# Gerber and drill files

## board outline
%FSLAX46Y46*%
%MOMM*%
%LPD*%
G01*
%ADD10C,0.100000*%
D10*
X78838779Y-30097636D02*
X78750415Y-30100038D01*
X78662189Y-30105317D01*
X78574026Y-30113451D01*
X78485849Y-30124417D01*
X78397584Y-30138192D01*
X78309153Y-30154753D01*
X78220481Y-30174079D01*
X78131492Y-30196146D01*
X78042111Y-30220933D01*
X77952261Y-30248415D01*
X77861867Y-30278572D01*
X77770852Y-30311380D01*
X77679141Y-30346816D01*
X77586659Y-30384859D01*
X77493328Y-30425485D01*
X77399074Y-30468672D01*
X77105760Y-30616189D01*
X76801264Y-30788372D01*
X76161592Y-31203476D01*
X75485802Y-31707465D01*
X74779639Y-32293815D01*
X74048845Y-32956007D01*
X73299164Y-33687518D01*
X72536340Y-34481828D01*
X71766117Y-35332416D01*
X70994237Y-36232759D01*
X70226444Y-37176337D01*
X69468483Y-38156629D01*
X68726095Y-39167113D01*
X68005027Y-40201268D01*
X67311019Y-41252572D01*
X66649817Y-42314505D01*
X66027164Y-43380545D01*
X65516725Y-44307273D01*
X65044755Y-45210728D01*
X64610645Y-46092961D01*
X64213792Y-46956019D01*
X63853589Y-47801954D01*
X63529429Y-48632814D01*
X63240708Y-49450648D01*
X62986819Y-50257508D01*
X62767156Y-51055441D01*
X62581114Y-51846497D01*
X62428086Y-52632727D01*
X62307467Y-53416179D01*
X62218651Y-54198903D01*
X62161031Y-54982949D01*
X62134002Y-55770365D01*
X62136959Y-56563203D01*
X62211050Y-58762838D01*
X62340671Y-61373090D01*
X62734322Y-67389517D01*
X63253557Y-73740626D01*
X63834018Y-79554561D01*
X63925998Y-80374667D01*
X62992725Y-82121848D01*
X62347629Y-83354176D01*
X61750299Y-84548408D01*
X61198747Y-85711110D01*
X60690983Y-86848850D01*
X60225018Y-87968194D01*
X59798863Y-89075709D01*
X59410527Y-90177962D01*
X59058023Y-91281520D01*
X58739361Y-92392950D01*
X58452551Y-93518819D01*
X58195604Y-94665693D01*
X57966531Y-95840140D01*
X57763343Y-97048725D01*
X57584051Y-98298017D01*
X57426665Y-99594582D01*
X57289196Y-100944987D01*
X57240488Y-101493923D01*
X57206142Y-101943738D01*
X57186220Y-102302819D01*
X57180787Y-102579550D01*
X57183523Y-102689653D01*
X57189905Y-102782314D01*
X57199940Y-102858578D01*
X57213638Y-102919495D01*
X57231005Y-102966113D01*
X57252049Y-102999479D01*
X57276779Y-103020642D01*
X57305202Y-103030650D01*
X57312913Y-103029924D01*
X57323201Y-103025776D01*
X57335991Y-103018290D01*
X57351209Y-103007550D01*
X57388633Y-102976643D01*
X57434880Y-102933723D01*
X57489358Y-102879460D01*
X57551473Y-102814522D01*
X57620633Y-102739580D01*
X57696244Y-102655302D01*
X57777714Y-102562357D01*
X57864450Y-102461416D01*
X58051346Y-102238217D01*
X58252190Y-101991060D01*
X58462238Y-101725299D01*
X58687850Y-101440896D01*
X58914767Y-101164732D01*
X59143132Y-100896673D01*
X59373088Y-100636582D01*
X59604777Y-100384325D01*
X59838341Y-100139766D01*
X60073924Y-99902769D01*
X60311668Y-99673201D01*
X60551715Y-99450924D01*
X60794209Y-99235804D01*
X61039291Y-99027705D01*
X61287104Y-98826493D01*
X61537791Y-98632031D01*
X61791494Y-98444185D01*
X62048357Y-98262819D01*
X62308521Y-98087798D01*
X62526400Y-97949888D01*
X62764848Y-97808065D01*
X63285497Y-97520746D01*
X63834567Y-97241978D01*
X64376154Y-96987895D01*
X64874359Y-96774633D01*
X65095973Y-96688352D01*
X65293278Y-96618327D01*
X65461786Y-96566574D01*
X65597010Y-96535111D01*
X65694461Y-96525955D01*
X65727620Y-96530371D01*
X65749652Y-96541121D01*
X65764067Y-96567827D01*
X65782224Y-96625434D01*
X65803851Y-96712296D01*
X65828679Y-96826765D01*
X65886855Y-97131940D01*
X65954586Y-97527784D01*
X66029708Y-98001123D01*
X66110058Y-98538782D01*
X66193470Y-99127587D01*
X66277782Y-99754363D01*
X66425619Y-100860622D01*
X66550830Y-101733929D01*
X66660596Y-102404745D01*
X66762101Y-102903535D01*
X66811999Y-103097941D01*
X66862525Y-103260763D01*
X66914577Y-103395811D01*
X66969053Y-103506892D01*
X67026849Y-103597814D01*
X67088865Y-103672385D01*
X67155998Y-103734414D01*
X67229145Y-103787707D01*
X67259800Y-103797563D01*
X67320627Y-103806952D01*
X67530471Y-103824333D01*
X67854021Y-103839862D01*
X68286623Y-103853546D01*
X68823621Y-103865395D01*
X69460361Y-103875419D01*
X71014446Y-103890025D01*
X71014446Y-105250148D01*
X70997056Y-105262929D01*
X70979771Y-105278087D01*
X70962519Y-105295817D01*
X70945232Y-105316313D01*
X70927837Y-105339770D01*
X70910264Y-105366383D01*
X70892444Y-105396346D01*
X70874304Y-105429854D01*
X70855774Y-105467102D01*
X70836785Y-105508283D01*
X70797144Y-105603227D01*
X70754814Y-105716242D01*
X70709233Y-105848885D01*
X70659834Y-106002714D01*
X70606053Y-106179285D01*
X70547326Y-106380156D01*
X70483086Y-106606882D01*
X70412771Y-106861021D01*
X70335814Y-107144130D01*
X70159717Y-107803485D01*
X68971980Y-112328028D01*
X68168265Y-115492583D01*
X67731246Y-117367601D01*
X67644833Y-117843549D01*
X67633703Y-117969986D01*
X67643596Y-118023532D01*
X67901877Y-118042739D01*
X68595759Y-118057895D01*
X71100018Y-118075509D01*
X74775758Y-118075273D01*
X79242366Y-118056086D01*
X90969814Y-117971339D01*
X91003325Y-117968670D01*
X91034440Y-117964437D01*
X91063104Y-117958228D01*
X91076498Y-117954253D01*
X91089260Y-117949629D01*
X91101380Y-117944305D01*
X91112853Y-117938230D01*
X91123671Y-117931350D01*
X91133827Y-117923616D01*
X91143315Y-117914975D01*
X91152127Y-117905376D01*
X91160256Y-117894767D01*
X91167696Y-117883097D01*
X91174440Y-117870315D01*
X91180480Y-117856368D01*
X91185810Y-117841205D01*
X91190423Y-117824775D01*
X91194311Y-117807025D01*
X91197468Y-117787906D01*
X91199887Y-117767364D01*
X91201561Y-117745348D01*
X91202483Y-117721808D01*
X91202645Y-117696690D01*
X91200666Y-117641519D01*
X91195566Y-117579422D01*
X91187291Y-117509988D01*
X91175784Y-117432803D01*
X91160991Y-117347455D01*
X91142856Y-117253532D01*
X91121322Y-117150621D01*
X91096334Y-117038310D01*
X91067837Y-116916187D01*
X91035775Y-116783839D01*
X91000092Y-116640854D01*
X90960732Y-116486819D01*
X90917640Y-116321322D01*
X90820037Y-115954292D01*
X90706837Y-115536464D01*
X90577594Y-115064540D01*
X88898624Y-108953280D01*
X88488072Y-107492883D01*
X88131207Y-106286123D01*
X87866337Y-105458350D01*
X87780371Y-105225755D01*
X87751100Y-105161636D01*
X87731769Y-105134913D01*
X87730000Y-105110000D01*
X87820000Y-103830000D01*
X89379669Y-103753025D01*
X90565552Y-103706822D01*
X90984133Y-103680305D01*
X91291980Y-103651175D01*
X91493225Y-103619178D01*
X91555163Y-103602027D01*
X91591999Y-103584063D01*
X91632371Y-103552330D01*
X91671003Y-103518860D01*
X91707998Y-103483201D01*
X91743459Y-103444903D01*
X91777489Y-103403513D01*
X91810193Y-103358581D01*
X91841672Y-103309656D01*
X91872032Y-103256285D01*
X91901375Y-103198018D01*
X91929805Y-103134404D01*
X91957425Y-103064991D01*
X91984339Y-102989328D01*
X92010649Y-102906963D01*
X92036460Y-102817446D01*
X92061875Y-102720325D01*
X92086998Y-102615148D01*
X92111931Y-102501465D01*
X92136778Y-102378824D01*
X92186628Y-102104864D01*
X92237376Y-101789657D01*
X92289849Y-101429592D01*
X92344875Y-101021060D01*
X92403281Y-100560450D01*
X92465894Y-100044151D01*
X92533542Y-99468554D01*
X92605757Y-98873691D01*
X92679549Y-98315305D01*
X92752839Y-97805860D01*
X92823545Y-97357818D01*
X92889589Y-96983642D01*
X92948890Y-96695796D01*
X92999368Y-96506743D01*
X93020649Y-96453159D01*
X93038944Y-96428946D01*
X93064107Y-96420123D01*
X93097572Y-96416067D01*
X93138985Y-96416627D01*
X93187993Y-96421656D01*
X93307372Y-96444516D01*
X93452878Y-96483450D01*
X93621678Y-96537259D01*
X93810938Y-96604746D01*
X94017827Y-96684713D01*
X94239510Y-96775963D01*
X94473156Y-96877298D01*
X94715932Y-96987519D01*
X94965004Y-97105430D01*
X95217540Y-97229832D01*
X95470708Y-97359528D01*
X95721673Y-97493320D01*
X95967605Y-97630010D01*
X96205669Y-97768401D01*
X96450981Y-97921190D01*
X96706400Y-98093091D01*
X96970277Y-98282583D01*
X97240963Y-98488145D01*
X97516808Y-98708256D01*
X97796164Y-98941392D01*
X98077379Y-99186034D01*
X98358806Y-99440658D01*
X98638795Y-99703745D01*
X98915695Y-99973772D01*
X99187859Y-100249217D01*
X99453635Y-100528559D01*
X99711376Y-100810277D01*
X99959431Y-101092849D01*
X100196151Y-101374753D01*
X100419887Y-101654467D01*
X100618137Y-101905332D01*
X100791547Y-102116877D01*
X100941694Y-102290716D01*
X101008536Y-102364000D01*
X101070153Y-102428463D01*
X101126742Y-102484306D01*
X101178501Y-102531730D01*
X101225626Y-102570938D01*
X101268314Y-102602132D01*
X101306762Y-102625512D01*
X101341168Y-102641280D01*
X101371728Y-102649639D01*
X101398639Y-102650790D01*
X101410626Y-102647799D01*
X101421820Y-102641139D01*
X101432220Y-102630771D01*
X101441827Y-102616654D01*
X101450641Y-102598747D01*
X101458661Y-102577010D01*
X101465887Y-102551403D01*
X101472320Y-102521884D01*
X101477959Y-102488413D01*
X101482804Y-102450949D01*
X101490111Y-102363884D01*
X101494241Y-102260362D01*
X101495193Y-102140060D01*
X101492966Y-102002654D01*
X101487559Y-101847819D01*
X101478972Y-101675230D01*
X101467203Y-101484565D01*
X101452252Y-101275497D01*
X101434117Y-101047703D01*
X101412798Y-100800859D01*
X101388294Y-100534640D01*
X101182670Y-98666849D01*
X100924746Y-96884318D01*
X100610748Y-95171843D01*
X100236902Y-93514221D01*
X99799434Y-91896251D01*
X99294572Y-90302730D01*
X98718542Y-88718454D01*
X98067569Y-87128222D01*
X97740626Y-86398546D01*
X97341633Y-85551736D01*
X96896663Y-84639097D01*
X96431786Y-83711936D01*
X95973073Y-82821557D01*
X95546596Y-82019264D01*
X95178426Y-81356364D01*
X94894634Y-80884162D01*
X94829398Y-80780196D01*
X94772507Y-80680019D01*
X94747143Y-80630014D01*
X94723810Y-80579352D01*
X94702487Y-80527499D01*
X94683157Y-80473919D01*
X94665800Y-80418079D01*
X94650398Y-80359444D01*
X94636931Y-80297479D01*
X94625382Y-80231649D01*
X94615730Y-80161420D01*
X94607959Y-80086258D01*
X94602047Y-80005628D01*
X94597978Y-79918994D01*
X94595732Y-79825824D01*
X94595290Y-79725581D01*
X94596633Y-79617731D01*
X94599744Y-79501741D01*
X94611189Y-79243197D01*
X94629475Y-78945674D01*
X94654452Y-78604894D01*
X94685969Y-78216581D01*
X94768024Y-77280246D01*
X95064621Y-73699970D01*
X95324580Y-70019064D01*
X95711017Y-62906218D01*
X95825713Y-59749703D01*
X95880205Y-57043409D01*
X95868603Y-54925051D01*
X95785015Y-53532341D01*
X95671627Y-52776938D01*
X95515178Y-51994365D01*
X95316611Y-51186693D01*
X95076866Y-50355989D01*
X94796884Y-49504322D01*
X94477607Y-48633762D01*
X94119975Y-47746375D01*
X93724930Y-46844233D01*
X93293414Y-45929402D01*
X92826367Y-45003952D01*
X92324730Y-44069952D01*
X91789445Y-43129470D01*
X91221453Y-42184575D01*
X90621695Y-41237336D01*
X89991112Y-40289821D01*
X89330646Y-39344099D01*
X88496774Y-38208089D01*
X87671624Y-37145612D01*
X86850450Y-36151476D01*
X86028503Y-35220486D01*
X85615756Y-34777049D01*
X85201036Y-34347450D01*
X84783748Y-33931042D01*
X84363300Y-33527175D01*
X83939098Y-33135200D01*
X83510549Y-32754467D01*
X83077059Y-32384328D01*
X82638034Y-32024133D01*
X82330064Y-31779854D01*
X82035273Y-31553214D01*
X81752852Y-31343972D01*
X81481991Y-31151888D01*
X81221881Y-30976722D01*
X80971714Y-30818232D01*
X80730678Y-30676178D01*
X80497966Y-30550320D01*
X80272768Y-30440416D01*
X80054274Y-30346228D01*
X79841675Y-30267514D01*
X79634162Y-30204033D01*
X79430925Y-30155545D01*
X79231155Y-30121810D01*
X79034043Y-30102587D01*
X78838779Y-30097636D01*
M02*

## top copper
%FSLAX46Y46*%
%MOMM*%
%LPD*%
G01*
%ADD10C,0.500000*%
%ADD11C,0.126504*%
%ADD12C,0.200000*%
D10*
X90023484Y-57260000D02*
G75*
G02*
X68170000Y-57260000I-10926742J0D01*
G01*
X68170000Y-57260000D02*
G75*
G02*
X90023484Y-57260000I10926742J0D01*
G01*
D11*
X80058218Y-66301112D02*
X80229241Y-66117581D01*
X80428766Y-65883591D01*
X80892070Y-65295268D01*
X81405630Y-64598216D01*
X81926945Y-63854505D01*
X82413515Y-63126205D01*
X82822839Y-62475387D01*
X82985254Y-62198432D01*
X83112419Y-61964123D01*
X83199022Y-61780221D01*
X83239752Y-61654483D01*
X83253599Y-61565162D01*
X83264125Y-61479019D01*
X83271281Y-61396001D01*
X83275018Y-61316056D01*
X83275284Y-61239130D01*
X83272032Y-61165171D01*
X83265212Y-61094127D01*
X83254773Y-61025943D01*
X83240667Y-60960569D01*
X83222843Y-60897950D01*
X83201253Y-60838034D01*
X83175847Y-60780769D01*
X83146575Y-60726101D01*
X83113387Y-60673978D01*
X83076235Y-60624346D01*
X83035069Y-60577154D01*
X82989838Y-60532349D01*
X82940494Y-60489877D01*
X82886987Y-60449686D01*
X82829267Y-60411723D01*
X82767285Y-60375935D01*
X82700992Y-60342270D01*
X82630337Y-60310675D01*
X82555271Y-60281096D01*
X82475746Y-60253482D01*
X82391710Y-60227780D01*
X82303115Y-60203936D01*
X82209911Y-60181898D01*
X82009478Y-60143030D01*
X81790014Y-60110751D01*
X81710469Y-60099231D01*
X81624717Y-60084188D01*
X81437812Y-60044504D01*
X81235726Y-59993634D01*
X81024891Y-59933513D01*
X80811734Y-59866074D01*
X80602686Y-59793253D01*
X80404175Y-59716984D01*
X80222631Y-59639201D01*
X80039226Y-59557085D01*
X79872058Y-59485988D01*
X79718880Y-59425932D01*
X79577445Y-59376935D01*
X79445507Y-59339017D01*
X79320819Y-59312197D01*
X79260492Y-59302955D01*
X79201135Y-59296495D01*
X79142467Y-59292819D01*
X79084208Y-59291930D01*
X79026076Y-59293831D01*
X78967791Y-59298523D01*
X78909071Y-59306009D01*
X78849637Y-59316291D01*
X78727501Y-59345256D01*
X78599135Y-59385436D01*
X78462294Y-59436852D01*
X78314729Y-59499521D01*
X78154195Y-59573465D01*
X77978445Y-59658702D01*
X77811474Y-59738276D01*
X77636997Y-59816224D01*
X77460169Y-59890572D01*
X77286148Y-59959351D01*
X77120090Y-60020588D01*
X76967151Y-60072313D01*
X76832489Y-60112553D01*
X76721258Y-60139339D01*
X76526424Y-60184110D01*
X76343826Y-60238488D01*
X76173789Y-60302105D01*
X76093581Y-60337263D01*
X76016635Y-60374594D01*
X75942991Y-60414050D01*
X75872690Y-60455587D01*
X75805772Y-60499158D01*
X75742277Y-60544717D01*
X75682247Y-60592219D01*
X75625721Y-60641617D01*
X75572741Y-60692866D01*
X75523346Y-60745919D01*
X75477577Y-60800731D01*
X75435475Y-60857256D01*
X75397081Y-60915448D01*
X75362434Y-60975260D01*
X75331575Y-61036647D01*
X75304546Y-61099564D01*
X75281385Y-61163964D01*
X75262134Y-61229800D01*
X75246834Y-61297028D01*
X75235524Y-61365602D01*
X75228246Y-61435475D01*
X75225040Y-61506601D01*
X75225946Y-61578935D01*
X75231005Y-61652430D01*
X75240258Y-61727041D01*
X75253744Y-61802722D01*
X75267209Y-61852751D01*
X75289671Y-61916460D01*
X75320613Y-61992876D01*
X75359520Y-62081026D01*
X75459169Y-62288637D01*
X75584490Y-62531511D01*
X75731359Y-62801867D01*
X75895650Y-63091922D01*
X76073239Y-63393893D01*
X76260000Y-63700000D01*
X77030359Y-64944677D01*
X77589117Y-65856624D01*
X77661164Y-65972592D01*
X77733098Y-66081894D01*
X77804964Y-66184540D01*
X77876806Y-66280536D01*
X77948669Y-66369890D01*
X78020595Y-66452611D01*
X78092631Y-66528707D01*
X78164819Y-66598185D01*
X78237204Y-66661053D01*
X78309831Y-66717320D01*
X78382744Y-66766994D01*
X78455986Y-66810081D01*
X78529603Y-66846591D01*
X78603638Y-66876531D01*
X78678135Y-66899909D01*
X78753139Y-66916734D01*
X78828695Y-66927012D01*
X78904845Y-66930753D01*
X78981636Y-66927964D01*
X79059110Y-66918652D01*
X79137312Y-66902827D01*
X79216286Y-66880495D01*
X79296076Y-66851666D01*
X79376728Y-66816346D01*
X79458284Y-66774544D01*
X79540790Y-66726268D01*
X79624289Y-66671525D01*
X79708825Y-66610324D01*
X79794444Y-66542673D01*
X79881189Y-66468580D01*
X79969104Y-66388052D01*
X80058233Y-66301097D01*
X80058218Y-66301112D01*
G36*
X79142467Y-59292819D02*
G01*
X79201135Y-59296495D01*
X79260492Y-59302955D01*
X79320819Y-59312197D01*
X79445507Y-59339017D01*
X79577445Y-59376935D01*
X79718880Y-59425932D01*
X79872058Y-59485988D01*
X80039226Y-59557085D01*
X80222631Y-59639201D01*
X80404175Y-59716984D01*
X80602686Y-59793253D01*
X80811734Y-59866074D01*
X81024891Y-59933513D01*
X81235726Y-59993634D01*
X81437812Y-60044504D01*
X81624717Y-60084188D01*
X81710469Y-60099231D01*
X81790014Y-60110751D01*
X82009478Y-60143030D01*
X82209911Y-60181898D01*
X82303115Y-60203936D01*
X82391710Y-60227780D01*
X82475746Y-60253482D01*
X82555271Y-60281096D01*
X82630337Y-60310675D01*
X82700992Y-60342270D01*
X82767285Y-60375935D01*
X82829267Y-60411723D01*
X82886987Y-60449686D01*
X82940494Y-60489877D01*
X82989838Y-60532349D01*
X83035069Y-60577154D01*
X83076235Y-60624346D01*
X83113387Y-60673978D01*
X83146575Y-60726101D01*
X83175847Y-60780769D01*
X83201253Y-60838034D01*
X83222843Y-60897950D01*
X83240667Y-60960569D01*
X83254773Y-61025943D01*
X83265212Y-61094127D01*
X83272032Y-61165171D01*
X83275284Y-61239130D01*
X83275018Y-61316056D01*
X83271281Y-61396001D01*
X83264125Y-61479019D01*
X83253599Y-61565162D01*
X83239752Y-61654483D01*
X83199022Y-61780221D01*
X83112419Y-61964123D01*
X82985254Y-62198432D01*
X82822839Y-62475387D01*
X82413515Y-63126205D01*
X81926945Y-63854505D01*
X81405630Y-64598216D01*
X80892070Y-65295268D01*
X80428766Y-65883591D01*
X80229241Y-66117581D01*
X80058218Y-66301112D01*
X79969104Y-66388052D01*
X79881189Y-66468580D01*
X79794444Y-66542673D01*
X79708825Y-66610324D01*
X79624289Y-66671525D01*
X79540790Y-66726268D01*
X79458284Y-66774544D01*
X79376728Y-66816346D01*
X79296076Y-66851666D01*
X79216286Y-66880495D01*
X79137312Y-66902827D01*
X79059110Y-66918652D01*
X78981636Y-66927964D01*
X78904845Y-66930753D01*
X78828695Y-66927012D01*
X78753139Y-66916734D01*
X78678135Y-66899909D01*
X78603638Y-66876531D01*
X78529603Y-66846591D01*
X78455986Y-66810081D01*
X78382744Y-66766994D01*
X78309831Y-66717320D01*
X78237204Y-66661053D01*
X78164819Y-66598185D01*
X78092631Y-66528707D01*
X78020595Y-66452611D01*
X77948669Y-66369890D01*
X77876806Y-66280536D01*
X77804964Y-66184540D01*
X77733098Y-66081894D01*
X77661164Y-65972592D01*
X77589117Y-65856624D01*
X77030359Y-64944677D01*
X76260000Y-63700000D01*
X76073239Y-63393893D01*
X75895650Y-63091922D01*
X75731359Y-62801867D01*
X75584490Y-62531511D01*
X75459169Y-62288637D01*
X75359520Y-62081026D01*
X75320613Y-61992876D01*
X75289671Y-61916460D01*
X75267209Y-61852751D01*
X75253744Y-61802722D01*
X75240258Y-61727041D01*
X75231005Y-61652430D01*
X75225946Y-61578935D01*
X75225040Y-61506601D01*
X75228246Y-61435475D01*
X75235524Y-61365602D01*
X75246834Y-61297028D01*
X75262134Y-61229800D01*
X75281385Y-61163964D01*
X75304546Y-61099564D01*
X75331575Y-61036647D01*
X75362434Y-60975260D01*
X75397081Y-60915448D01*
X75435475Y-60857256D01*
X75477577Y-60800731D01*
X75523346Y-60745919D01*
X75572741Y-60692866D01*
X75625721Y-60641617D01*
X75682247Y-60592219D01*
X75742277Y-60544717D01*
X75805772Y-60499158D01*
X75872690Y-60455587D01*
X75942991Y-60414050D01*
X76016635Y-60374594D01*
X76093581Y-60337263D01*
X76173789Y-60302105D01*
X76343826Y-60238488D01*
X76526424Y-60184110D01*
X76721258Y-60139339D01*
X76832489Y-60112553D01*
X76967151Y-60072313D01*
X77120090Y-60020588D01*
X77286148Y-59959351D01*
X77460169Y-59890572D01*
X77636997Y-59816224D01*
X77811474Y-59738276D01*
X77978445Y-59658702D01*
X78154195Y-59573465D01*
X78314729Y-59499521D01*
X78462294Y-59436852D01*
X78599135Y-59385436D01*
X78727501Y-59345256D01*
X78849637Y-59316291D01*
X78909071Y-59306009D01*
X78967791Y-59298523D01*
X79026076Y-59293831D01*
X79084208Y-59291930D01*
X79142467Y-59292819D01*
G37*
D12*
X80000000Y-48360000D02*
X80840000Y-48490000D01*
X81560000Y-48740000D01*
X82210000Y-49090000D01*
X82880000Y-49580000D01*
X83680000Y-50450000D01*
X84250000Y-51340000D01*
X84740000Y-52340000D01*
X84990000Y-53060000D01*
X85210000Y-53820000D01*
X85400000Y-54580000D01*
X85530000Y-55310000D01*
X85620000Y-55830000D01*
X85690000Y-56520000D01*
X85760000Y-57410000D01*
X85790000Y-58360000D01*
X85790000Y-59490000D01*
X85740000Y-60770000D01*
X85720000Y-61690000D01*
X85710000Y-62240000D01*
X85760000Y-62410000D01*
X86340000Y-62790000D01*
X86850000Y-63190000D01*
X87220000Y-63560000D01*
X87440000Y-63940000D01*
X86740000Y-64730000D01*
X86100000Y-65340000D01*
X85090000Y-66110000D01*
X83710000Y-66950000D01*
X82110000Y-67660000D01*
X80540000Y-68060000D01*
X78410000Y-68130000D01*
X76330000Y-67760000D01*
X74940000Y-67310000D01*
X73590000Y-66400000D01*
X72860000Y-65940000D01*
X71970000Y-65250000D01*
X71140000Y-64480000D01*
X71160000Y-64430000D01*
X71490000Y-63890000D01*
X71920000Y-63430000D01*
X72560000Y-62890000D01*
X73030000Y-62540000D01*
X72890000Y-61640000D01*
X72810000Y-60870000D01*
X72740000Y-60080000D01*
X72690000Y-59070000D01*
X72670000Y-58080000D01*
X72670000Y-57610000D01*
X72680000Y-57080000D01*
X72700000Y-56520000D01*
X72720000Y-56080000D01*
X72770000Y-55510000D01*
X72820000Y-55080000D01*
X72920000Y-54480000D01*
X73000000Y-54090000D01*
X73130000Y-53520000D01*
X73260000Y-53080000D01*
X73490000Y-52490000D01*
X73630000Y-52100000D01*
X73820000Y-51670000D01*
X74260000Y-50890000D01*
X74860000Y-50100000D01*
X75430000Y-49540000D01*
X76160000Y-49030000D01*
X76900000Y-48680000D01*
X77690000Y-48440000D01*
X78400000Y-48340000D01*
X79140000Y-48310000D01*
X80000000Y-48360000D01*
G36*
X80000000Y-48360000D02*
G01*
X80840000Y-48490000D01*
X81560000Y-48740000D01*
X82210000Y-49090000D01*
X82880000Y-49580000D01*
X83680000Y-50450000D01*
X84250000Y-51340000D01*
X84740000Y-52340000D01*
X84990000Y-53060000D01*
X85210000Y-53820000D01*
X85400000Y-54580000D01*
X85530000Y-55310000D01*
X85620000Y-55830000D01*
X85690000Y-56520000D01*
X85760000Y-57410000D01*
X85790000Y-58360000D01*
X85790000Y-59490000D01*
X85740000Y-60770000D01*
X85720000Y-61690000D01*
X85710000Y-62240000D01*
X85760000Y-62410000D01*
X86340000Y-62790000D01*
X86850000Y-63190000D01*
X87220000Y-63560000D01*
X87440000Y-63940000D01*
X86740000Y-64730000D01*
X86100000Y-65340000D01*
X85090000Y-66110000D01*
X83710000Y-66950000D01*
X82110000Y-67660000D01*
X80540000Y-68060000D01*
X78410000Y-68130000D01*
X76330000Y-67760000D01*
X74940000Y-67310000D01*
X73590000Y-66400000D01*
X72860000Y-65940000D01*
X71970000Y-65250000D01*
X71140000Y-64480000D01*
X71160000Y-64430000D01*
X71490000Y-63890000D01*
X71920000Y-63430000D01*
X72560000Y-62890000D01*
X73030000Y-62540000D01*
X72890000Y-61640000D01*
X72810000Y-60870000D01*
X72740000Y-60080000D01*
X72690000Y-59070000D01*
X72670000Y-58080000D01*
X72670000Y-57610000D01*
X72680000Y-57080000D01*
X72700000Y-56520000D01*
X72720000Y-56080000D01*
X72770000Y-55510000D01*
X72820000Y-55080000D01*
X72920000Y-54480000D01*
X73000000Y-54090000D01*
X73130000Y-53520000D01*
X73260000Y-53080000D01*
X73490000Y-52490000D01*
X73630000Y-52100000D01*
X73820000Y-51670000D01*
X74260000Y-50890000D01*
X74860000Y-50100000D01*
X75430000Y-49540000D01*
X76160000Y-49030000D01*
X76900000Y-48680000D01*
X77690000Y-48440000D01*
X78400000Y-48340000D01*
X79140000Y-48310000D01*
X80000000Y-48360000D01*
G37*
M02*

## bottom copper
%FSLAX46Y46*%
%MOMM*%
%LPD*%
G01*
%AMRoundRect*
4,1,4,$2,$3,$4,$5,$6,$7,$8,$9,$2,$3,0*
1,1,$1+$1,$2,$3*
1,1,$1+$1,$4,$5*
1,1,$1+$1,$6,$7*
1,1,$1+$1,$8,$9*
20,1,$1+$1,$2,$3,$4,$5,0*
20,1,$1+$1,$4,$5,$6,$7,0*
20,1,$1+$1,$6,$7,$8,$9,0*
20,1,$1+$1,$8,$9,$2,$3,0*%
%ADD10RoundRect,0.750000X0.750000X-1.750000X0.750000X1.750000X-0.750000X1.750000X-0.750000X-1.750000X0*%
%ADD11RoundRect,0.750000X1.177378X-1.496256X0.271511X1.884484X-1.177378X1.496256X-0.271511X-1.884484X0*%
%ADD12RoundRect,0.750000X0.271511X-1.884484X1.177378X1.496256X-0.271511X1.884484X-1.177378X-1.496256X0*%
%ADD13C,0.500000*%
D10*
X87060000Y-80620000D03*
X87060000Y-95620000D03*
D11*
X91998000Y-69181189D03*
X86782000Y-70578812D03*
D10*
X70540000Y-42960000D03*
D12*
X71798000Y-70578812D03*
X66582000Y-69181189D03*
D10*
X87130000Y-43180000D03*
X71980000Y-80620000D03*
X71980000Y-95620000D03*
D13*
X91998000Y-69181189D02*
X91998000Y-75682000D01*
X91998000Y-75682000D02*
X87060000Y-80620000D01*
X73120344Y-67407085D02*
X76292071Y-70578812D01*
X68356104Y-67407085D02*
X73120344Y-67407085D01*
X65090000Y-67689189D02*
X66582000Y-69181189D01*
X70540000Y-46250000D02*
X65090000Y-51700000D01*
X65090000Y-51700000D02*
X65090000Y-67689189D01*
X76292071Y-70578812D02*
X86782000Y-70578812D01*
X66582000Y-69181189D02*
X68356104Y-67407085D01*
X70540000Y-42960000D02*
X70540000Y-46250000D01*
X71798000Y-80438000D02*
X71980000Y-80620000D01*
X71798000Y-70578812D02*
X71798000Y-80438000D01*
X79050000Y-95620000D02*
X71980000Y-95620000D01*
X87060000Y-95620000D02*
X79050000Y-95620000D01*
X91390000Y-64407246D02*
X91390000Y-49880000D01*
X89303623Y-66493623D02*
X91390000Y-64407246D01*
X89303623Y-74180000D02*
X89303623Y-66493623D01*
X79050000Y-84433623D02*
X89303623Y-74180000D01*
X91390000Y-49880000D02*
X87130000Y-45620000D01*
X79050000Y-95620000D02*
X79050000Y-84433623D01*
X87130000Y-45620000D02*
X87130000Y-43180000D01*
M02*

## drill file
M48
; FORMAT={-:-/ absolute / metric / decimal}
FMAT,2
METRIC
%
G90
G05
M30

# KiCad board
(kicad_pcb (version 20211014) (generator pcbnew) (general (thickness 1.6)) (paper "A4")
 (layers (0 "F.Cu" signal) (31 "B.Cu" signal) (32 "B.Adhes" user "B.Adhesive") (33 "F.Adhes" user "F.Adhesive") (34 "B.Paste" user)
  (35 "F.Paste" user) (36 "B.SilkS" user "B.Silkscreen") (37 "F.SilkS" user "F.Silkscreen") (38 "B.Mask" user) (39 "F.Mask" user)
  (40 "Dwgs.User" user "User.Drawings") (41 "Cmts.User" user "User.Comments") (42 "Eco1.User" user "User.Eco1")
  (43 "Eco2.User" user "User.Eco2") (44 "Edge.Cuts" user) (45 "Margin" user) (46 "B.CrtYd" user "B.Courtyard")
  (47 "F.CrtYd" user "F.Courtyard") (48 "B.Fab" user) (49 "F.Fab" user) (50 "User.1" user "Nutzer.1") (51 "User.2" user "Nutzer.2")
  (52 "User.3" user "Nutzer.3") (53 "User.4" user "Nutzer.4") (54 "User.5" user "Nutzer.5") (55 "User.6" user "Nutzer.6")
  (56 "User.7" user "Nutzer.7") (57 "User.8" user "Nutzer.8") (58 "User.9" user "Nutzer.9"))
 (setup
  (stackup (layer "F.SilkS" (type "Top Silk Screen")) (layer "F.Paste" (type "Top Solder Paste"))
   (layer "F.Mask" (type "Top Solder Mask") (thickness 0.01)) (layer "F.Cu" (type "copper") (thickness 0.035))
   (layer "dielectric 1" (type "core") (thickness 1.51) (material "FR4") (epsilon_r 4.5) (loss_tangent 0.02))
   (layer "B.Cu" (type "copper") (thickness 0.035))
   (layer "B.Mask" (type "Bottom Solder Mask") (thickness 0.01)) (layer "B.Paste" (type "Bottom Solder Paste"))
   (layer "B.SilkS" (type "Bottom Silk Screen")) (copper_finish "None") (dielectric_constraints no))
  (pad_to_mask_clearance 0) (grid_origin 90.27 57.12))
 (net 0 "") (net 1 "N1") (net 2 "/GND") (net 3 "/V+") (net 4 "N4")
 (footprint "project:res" (layer "B.Cu") (at 87.06 88.12 180)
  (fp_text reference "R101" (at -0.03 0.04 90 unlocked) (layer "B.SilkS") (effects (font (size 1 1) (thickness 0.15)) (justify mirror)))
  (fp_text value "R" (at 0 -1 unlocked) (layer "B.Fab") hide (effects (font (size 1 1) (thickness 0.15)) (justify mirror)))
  (pad "1" smd roundrect (at 0 7.5 90) (size 5 3) (layers "B.Cu" "B.Paste" "B.Mask") (roundrect_rratio 0.25) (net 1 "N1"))
  (pad "2" smd roundrect (at 0 -7.5 90) (size 5 3) (layers "B.Cu" "B.Paste" "B.Mask") (roundrect_rratio 0.25) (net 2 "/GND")))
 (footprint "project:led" (layer "B.Cu") (at 91.967041 70.224761 -165)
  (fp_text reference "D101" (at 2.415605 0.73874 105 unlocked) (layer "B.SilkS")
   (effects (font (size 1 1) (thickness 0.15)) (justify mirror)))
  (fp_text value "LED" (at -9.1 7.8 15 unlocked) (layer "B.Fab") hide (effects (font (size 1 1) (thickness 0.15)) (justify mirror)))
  (pad "1" smd roundrect (at -0.3 1 105) (size 5 3) (layers "B.Cu" "B.Paste" "B.Mask") (roundrect_rratio 0.25) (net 1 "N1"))
  (pad "2" smd roundrect (at 5.1 1 105) (size 5 3) (layers "B.Cu" "B.Paste" "B.Mask") (roundrect_rratio 0.25) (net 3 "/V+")))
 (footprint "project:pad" (layer "B.Cu") (at 70.74 42.96 180)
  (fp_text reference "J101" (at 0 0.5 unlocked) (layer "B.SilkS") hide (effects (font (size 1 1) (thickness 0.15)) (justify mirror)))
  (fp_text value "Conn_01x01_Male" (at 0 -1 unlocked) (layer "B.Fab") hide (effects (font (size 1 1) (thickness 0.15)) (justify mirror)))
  (pad "1" smd roundrect (at 0.2 0 90) (size 5 3) (layers "B.Cu" "B.Paste" "B.Mask") (roundrect_rratio 0.25) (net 3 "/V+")))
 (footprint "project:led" (layer "B.Cu") (at 71.249403 71.467092 165)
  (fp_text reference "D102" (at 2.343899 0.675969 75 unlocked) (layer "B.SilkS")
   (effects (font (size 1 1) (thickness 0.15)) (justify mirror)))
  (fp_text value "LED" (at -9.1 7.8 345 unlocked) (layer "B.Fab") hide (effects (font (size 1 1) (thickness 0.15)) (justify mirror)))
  (pad "1" smd roundrect (at -0.3 1 75) (size 5 3) (layers "B.Cu" "B.Paste" "B.Mask") (roundrect_rratio 0.25) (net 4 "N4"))
  (pad "2" smd roundrect (at 5.1 1 75) (size 5 3) (layers "B.Cu" "B.Paste" "B.Mask") (roundrect_rratio 0.25) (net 3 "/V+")))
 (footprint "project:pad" (layer "B.Cu") (at 87.33 43.18 180)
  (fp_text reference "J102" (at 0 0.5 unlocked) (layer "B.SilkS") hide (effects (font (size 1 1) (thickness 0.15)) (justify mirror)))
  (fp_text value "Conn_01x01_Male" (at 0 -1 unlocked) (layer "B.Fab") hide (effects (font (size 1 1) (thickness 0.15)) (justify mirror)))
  (pad "1" smd roundrect (at 0.2 0 90) (size 5 3) (layers "B.Cu" "B.Paste" "B.Mask") (roundrect_rratio 0.25) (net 2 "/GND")))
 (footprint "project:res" (layer "B.Cu") (at 71.98 88.12 180)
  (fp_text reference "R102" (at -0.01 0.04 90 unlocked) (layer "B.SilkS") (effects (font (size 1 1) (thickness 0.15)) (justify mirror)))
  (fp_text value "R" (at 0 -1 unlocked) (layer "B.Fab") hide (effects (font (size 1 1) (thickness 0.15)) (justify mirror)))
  (pad "1" smd roundrect (at 0 7.5 90) (size 5 3) (layers "B.Cu" "B.Paste" "B.Mask") (roundrect_rratio 0.25) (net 4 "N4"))
  (pad "2" smd roundrect (at 0 -7.5 90) (size 5 3) (layers "B.Cu" "B.Paste" "B.Mask") (roundrect_rratio 0.25) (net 2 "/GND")))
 (gr_circle (center 79.096742 57.26) (end 90.023484 57.26) (layer "F.Cu") (width 0.5) (fill none))
 (gr_poly
  (pts (xy 80.058218 66.301112) (xy 80.229241 66.117581) (xy 80.428766 65.883591) (xy 80.89207 65.295268) (xy 81.40563 64.598216)
   (xy 81.926945 63.854505) (xy 82.413515 63.126205) (xy 82.822839 62.475387) (xy 82.985254 62.198432) (xy 83.112419 61.964123)
   (xy 83.199022 61.780221) (xy 83.239752 61.654483) (xy 83.253599 61.565162) (xy 83.264125 61.479019) (xy 83.271281 61.396001)
   (xy 83.275018 61.316056) (xy 83.275284 61.23913) (xy 83.272032 61.165171) (xy 83.265212 61.094127) (xy 83.254773 61.025943)
   (xy 83.240667 60.960569) (xy 83.222843 60.89795) (xy 83.201253 60.838034) (xy 83.175847 60.780769) (xy 83.146575 60.726101)
   (xy 83.113387 60.673978) (xy 83.076235 60.624346) (xy 83.035069 60.577154) (xy 82.989838 60.532349) (xy 82.940494 60.489877)
   (xy 82.886987 60.449686) (xy 82.829267 60.411723) (xy 82.767285 60.375935) (xy 82.700992 60.34227) (xy 82.630337 60.310675)
   (xy 82.555271 60.281096) (xy 82.475746 60.253482) (xy 82.39171 60.22778) (xy 82.303115 60.203936) (xy 82.209911 60.181898)
   (xy 82.009478 60.14303) (xy 81.790014 60.110751) (xy 81.710469 60.099231) (xy 81.624717 60.084188) (xy 81.437812 60.044504)
   (xy 81.235726 59.993634) (xy 81.024891 59.933513) (xy 80.811734 59.866074) (xy 80.602686 59.793253) (xy 80.404175 59.716984)
   (xy 80.222631 59.639201) (xy 80.039226 59.557085) (xy 79.872058 59.485988) (xy 79.71888 59.425932) (xy 79.577445 59.376935)
   (xy 79.445507 59.339017) (xy 79.320819 59.312197) (xy 79.260492 59.302955) (xy 79.201135 59.296495) (xy 79.142467 59.292819)
   (xy 79.084208 59.29193) (xy 79.026076 59.293831) (xy 78.967791 59.298523) (xy 78.909071 59.306009) (xy 78.849637 59.316291)
   (xy 78.727501 59.345256) (xy 78.599135 59.385436) (xy 78.462294 59.436852) (xy 78.314729 59.499521) (xy 78.154195 59.573465)
   (xy 77.978445 59.658702) (xy 77.811474 59.738276) (xy 77.636997 59.816224) (xy 77.460169 59.890572) (xy 77.286148 59.959351)
   (xy 77.12009 60.020588) (xy 76.967151 60.072313) (xy 76.832489 60.112553) (xy 76.721258 60.139339) (xy 76.526424 60.18411)
   (xy 76.343826 60.238488) (xy 76.173789 60.302105) (xy 76.093581 60.337263) (xy 76.016635 60.374594) (xy 75.942991 60.41405)
   (xy 75.87269 60.455587) (xy 75.805772 60.499158) (xy 75.742277 60.544717) (xy 75.682247 60.592219) (xy 75.625721 60.641617)
   (xy 75.572741 60.692866) (xy 75.523346 60.745919) (xy 75.477577 60.800731) (xy 75.435475 60.857256) (xy 75.397081 60.915448)
   (xy 75.362434 60.97526) (xy 75.331575 61.036647) (xy 75.304546 61.099564) (xy 75.281385 61.163964) (xy 75.262134 61.2298)
   (xy 75.246834 61.297028) (xy 75.235524 61.365602) (xy 75.228246 61.435475) (xy 75.22504 61.506601) (xy 75.225946 61.578935)
   (xy 75.231005 61.65243) (xy 75.240258 61.727041) (xy 75.253744 61.802722) (xy 75.267209 61.852751) (xy 75.289671 61.91646)
   (xy 75.320613 61.992876) (xy 75.35952 62.081026) (xy 75.459169 62.288637) (xy 75.58449 62.531511) (xy 75.731359 62.801867)
   (xy 75.89565 63.091922) (xy 76.073239 63.393893) (xy 76.26 63.7) (xy 77.030359 64.944677) (xy 77.589117 65.856624)
   (xy 77.661164 65.972592) (xy 77.733098 66.081894) (xy 77.804964 66.18454) (xy 77.876806 66.280536) (xy 77.948669 66.36989)
   (xy 78.020595 66.452611) (xy 78.092631 66.528707) (xy 78.164819 66.598185) (xy 78.237204 66.661053) (xy 78.309831 66.71732)
   (xy 78.382744 66.766994) (xy 78.455986 66.810081) (xy 78.529603 66.846591) (xy 78.603638 66.876531) (xy 78.678135 66.899909)
   (xy 78.753139 66.916734) (xy 78.828695 66.927012) (xy 78.904845 66.930753) (xy 78.981636 66.927964) (xy 79.05911 66.918652)
   (xy 79.137312 66.902827) (xy 79.216286 66.880495) (xy 79.296076 66.851666) (xy 79.376728 66.816346) (xy 79.458284 66.774544)
   (xy 79.54079 66.726268) (xy 79.624289 66.671525) (xy 79.708825 66.610324) (xy 79.794444 66.542673) (xy 79.881189 66.46858)
   (xy 79.969104 66.388052) (xy 80.058233 66.301097) (xy 80.058218 66.301112))
  (layer "F.Cu") (width 0.126504) (fill solid))
 (gr_poly
  (pts (xy 80 48.36) (xy 80.84 48.49) (xy 81.56 48.74) (xy 82.21 49.09) (xy 82.88 49.58) (xy 83.68 50.45) (xy 84.25 51.34) (xy 84.74 52.34)
   (xy 84.99 53.06) (xy 85.21 53.82) (xy 85.4 54.58) (xy 85.53 55.31) (xy 85.62 55.83) (xy 85.69 56.52) (xy 85.76 57.41) (xy 85.79 58.36)
   (xy 85.79 59.49) (xy 85.74 60.77) (xy 85.72 61.69) (xy 85.71 62.24) (xy 85.76 62.41) (xy 86.34 62.79) (xy 86.85 63.19) (xy 87.22 63.56)
   (xy 87.44 63.94) (xy 86.74 64.73) (xy 86.1 65.34) (xy 85.09 66.11) (xy 83.71 66.95) (xy 82.11 67.66) (xy 80.54 68.06) (xy 78.41 68.13)
   (xy 76.33 67.76) (xy 74.94 67.31) (xy 73.59 66.4) (xy 72.86 65.94) (xy 71.97 65.25) (xy 71.14 64.48) (xy 71.16 64.43) (xy 71.49 63.89)
   (xy 71.92 63.43) (xy 72.56 62.89) (xy 73.03 62.54) (xy 72.89 61.64) (xy 72.81 60.87) (xy 72.74 60.08) (xy 72.69 59.07) (xy 72.67 58.08)
   (xy 72.67 57.61) (xy 72.68 57.08) (xy 72.7 56.52) (xy 72.72 56.08) (xy 72.77 55.51) (xy 72.82 55.08) (xy 72.92 54.48) (xy 73 54.09)
   (xy 73.13 53.52) (xy 73.26 53.08) (xy 73.49 52.49) (xy 73.63 52.1) (xy 73.82 51.67) (xy 74.26 50.89) (xy 74.86 50.1) (xy 75.43 49.54)
   (xy 76.16 49.03) (xy 76.9 48.68) (xy 77.69 48.44) (xy 78.4 48.34) (xy 79.14 48.31))
  (layer "F.Cu") (width 0.2) (fill solid))
 (gr_poly
  (pts (xy 78.838779 30.097636) (xy 78.750415 30.100038) (xy 78.662189 30.105317) (xy 78.574026 30.113451) (xy 78.485849 30.124417)
   (xy 78.397584 30.138192) (xy 78.309153 30.154753) (xy 78.220481 30.174079) (xy 78.131492 30.196146) (xy 78.042111 30.220933)
   (xy 77.952261 30.248415) (xy 77.861867 30.278572) (xy 77.770852 30.31138) (xy 77.679141 30.346816) (xy 77.586659 30.384859)
   (xy 77.493328 30.425485) (xy 77.399074 30.468672) (xy 77.10576 30.616189) (xy 76.801264 30.788372) (xy 76.161592 31.203476)
   (xy 75.485802 31.707465) (xy 74.779639 32.293815) (xy 74.048845 32.956007) (xy 73.299164 33.687518) (xy 72.53634 34.481828)
   (xy 71.766117 35.332416) (xy 70.994237 36.232759) (xy 70.226444 37.176337) (xy 69.468483 38.156629) (xy 68.726095 39.167113)
   (xy 68.005027 40.201268) (xy 67.311019 41.252572) (xy 66.649817 42.314505) (xy 66.027164 43.380545) (xy 65.516725 44.307273)
   (xy 65.044755 45.210728) (xy 64.610645 46.092961) (xy 64.213792 46.956019) (xy 63.853589 47.801954) (xy 63.529429 48.632814)
   (xy 63.240708 49.450648) (xy 62.986819 50.257508) (xy 62.767156 51.055441) (xy 62.581114 51.846497) (xy 62.428086 52.632727)
   (xy 62.307467 53.416179) (xy 62.218651 54.198903) (xy 62.161031 54.982949) (xy 62.134002 55.770365) (xy 62.136959 56.563203)
   (xy 62.21105 58.762838) (xy 62.340671 61.37309) (xy 62.734322 67.389517) (xy 63.253557 73.740626) (xy 63.834018 79.554561)
   (xy 63.925998 80.374667) (xy 62.992725 82.121848) (xy 62.347629 83.354176) (xy 61.750299 84.548408) (xy 61.198747 85.71111)
   (xy 60.690983 86.84885) (xy 60.225018 87.968194) (xy 59.798863 89.075709) (xy 59.410527 90.177962) (xy 59.058023 91.28152)
   (xy 58.739361 92.39295) (xy 58.452551 93.518819) (xy 58.195604 94.665693) (xy 57.966531 95.84014) (xy 57.763343 97.048725)
   (xy 57.584051 98.298017) (xy 57.426665 99.594582) (xy 57.289196 100.944987) (xy 57.240488 101.493923) (xy 57.206142 101.943738)
   (xy 57.18622 102.302819) (xy 57.180787 102.57955) (xy 57.183523 102.689653) (xy 57.189905 102.782314) (xy 57.19994 102.858578)
   (xy 57.213638 102.919495) (xy 57.231005 102.966113) (xy 57.252049 102.999479) (xy 57.276779 103.020642) (xy 57.305202 103.03065)
   (xy 57.312913 103.029924) (xy 57.323201 103.025776) (xy 57.335991 103.01829) (xy 57.351209 103.00755) (xy 57.388633 102.976643)
   (xy 57.43488 102.933723) (xy 57.489358 102.87946) (xy 57.551473 102.814522) (xy 57.620633 102.73958) (xy 57.696244 102.655302)
   (xy 57.777714 102.562357) (xy 57.86445 102.461416) (xy 58.051346 102.238217) (xy 58.25219 101.99106) (xy 58.462238 101.725299)
   (xy 58.68785 101.440896) (xy 58.914767 101.164732) (xy 59.143132 100.896673) (xy 59.373088 100.636582) (xy 59.604777 100.384325)
   (xy 59.838341 100.139766) (xy 60.073924 99.902769) (xy 60.311668 99.673201) (xy 60.551715 99.450924) (xy 60.794209 99.235804)
   (xy 61.039291 99.027705) (xy 61.287104 98.826493) (xy 61.537791 98.632031) (xy 61.791494 98.444185) (xy 62.048357 98.262819)
   (xy 62.308521 98.087798) (xy 62.5264 97.949888) (xy 62.764848 97.808065) (xy 63.285497 97.520746) (xy 63.834567 97.241978)
   (xy 64.376154 96.987895) (xy 64.874359 96.774633) (xy 65.095973 96.688352) (xy 65.293278 96.618327) (xy 65.461786 96.566574)
   (xy 65.59701 96.535111) (xy 65.694461 96.525955) (xy 65.72762 96.530371) (xy 65.749652 96.541121) (xy 65.764067 96.567827)
   (xy 65.782224 96.625434) (xy 65.803851 96.712296) (xy 65.828679 96.826765) (xy 65.886855 97.13194) (xy 65.954586 97.527784)
   (xy 66.029708 98.001123) (xy 66.110058 98.538782) (xy 66.19347 99.127587) (xy 66.277782 99.754363) (xy 66.425619 100.860622)
   (xy 66.55083 101.733929) (xy 66.660596 102.404745) (xy 66.762101 102.903535) (xy 66.811999 103.097941) (xy 66.862525 103.260763)
   (xy 66.914577 103.395811) (xy 66.969053 103.506892) (xy 67.026849 103.597814) (xy 67.088865 103.672385) (xy 67.155998 103.734414)
   (xy 67.229145 103.787707) (xy 67.2598 103.797563) (xy 67.320627 103.806952) (xy 67.530471 103.824333) (xy 67.854021 103.839862)
   (xy 68.286623 103.853546) (xy 68.823621 103.865395) (xy 69.460361 103.875419) (xy 71.014446 103.890025) (xy 71.014446 105.250148)
   (xy 70.997056 105.262929) (xy 70.979771 105.278087) (xy 70.962519 105.295817) (xy 70.945232 105.316313) (xy 70.927837 105.33977)
   (xy 70.910264 105.366383) (xy 70.892444 105.396346) (xy 70.874304 105.429854) (xy 70.855774 105.467102) (xy 70.836785 105.508283)
   (xy 70.797144 105.603227) (xy 70.754814 105.716242) (xy 70.709233 105.848885) (xy 70.659834 106.002714) (xy 70.606053 106.179285)
   (xy 70.547326 106.380156) (xy 70.483086 106.606882) (xy 70.412771 106.861021) (xy 70.335814 107.14413) (xy 70.159717 107.803485)
   (xy 68.97198 112.328028) (xy 68.168265 115.492583) (xy 67.731246 117.367601) (xy 67.644833 117.843549) (xy 67.633703 117.969986)
   (xy 67.643596 118.023532) (xy 67.901877 118.042739) (xy 68.595759 118.057895) (xy 71.100018 118.075509) (xy 74.775758 118.075273)
   (xy 79.242366 118.056086) (xy 90.969814 117.971339) (xy 91.003325 117.96867) (xy 91.03444 117.964437) (xy 91.063104 117.958228)
   (xy 91.076498 117.954253) (xy 91.08926 117.949629) (xy 91.10138 117.944305) (xy 91.112853 117.93823) (xy 91.123671 117.93135)
   (xy 91.133827 117.923616) (xy 91.143315 117.914975) (xy 91.152127 117.905376) (xy 91.160256 117.894767) (xy 91.167696 117.883097)
   (xy 91.17444 117.870315) (xy 91.18048 117.856368) (xy 91.18581 117.841205) (xy 91.190423 117.824775) (xy 91.194311 117.807025)
   (xy 91.197468 117.787906) (xy 91.199887 117.767364) (xy 91.201561 117.745348) (xy 91.202483 117.721808) (xy 91.202645 117.69669)
   (xy 91.200666 117.641519) (xy 91.195566 117.579422) (xy 91.187291 117.509988) (xy 91.175784 117.432803) (xy 91.160991 117.347455)
   (xy 91.142856 117.253532) (xy 91.121322 117.150621) (xy 91.096334 117.03831) (xy 91.067837 116.916187) (xy 91.035775 116.783839)
   (xy 91.000092 116.640854) (xy 90.960732 116.486819) (xy 90.91764 116.321322) (xy 90.820037 115.954292) (xy 90.706837 115.536464)
   (xy 90.577594 115.06454) (xy 88.898624 108.95328) (xy 88.488072 107.492883) (xy 88.131207 106.286123) (xy 87.866337 105.45835)
   (xy 87.780371 105.225755) (xy 87.7511 105.161636) (xy 87.731769 105.134913) (xy 87.73 105.11) (xy 87.82 103.83) (xy 89.379669 103.753025)
   (xy 90.565552 103.706822) (xy 90.984133 103.680305) (xy 91.29198 103.651175) (xy 91.493225 103.619178) (xy 91.555163 103.602027)
   (xy 91.591999 103.584063) (xy 91.632371 103.55233) (xy 91.671003 103.51886) (xy 91.707998 103.483201) (xy 91.743459 103.444903)
   (xy 91.777489 103.403513) (xy 91.810193 103.358581) (xy 91.841672 103.309656) (xy 91.872032 103.256285) (xy 91.901375 103.198018)
   (xy 91.929805 103.134404) (xy 91.957425 103.064991) (xy 91.984339 102.989328) (xy 92.010649 102.906963) (xy 92.03646 102.817446)
   (xy 92.061875 102.720325) (xy 92.086998 102.615148) (xy 92.111931 102.501465) (xy 92.136778 102.378824) (xy 92.186628 102.104864)
   (xy 92.237376 101.789657) (xy 92.289849 101.429592) (xy 92.344875 101.02106) (xy 92.403281 100.56045) (xy 92.465894 100.044151)
   (xy 92.533542 99.468554) (xy 92.605757 98.873691) (xy 92.679549 98.315305) (xy 92.752839 97.80586) (xy 92.823545 97.357818)
   (xy 92.889589 96.983642) (xy 92.94889 96.695796) (xy 92.999368 96.506743) (xy 93.020649 96.453159) (xy 93.038944 96.428946)
   (xy 93.064107 96.420123) (xy 93.097572 96.416067) (xy 93.138985 96.416627) (xy 93.187993 96.421656) (xy 93.307372 96.444516)
   (xy 93.452878 96.48345) (xy 93.621678 96.537259) (xy 93.810938 96.604746) (xy 94.017827 96.684713) (xy 94.23951 96.775963)
   (xy 94.473156 96.877298) (xy 94.715932 96.987519) (xy 94.965004 97.10543) (xy 95.21754 97.229832) (xy 95.470708 97.359528)
   (xy 95.721673 97.49332) (xy 95.967605 97.63001) (xy 96.205669 97.768401) (xy 96.450981 97.92119) (xy 96.7064 98.093091)
   (xy 96.970277 98.282583) (xy 97.240963 98.488145) (xy 97.516808 98.708256) (xy 97.796164 98.941392) (xy 98.077379 99.186034)
   (xy 98.358806 99.440658) (xy 98.638795 99.703745) (xy 98.915695 99.973772) (xy 99.187859 100.249217) (xy 99.453635 100.528559)
   (xy 99.711376 100.810277) (xy 99.959431 101.092849) (xy 100.196151 101.374753) (xy 100.419887 101.654467) (xy 100.618137 101.905332)
   (xy 100.791547 102.116877) (xy 100.941694 102.290716) (xy 101.008536 102.364) (xy 101.070153 102.428463) (xy 101.126742 102.484306)
   (xy 101.178501 102.53173) (xy 101.225626 102.570938) (xy 101.268314 102.602132) (xy 101.306762 102.625512) (xy 101.341168 102.64128)
   (xy 101.371728 102.649639) (xy 101.398639 102.65079) (xy 101.410626 102.647799) (xy 101.42182 102.641139) (xy 101.43222 102.630771)
   (xy 101.441827 102.616654) (xy 101.450641 102.598747) (xy 101.458661 102.57701) (xy 101.465887 102.551403) (xy 101.47232 102.521884)
   (xy 101.477959 102.488413) (xy 101.482804 102.450949) (xy 101.490111 102.363884) (xy 101.494241 102.260362) (xy 101.495193 102.14006)
   (xy 101.492966 102.002654) (xy 101.487559 101.847819) (xy 101.478972 101.67523) (xy 101.467203 101.484565) (xy 101.452252 101.275497)
   (xy 101.434117 101.047703) (xy 101.412798 100.800859) (xy 101.388294 100.53464) (xy 101.18267 98.666849) (xy 100.924746 96.884318)
   (xy 100.610748 95.171843) (xy 100.236902 93.514221) (xy 99.799434 91.896251) (xy 99.294572 90.30273) (xy 98.718542 88.718454)
   (xy 98.067569 87.128222) (xy 97.740626 86.398546) (xy 97.341633 85.551736) (xy 96.896663 84.639097) (xy 96.431786 83.711936)
   (xy 95.973073 82.821557) (xy 95.546596 82.019264) (xy 95.178426 81.356364) (xy 94.894634 80.884162) (xy 94.829398 80.780196)
   (xy 94.772507 80.680019) (xy 94.747143 80.630014) (xy 94.72381 80.579352) (xy 94.702487 80.527499) (xy 94.683157 80.473919)
   (xy 94.6658 80.418079) (xy 94.650398 80.359444) (xy 94.636931 80.297479) (xy 94.625382 80.231649) (xy 94.61573 80.16142)
   (xy 94.607959 80.086258) (xy 94.602047 80.005628) (xy 94.597978 79.918994) (xy 94.595732 79.825824) (xy 94.59529 79.725581)
   (xy 94.596633 79.617731) (xy 94.599744 79.501741) (xy 94.611189 79.243197) (xy 94.629475 78.945674) (xy 94.654452 78.604894)
   (xy 94.685969 78.216581) (xy 94.768024 77.280246) (xy 95.064621 73.69997) (xy 95.32458 70.019064) (xy 95.711017 62.906218)
   (xy 95.825713 59.749703) (xy 95.880205 57.043409) (xy 95.868603 54.925051) (xy 95.785015 53.532341) (xy 95.671627 52.776938)
   (xy 95.515178 51.994365) (xy 95.316611 51.186693) (xy 95.076866 50.355989) (xy 94.796884 49.504322) (xy 94.477607 48.633762)
   (xy 94.119975 47.746375) (xy 93.72493 46.844233) (xy 93.293414 45.929402) (xy 92.826367 45.003952) (xy 92.32473 44.069952)
   (xy 91.789445 43.12947) (xy 91.221453 42.184575) (xy 90.621695 41.237336) (xy 89.991112 40.289821) (xy 89.330646 39.344099)
   (xy 88.496774 38.208089) (xy 87.671624 37.145612) (xy 86.85045 36.151476) (xy 86.028503 35.220486) (xy 85.615756 34.777049)
   (xy 85.201036 34.34745) (xy 84.783748 33.931042) (xy 84.3633 33.527175) (xy 83.939098 33.1352) (xy 83.510549 32.754467)
   (xy 83.077059 32.384328) (xy 82.638034 32.024133) (xy 82.330064 31.779854) (xy 82.035273 31.553214) (xy 81.752852 31.343972)
   (xy 81.481991 31.151888) (xy 81.221881 30.976722) (xy 80.971714 30.818232) (xy 80.730678 30.676178) (xy 80.497966 30.55032)
   (xy 80.272768 30.440416) (xy 80.054274 30.346228) (xy 79.841675 30.267514) (xy 79.634162 30.204033) (xy 79.430925 30.155545)
   (xy 79.231155 30.12181) (xy 79.034043 30.102587) (xy 78.838779 30.097636))
  (layer "Edge.Cuts") (width 0.1) (fill none))
 (segment (start 91.998 69.181189) (end 91.998 75.682) (width 0.5) (layer "B.Cu") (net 1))
 (segment (start 91.998 75.682) (end 87.06 80.62) (width 0.5) (layer "B.Cu") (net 1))
 (segment (start 73.120344 67.407085) (end 76.292071 70.578812) (width 0.5) (layer "B.Cu") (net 3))
 (segment (start 68.356104 67.407085) (end 73.120344 67.407085) (width 0.5) (layer "B.Cu") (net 3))
 (segment (start 65.09 67.689189) (end 66.582 69.181189) (width 0.5) (layer "B.Cu") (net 3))
 (segment (start 70.54 46.25) (end 65.09 51.7) (width 0.5) (layer "B.Cu") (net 3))
 (segment (start 65.09 51.7) (end 65.09 67.689189) (width 0.5) (layer "B.Cu") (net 3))
 (segment (start 76.292071 70.578812) (end 86.782 70.578812) (width 0.5) (layer "B.Cu") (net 3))
 (segment (start 66.582 69.181189) (end 68.356104 67.407085) (width 0.5) (layer "B.Cu") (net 3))
 (segment (start 70.54 42.96) (end 70.54 46.25) (width 0.5) (layer "B.Cu") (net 3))
 (segment (start 71.798 80.438) (end 71.98 80.62) (width 0.5) (layer "B.Cu") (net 4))
 (segment (start 71.798 70.578812) (end 71.798 80.438) (width 0.5) (layer "B.Cu") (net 4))
 (segment (start 79.05 95.62) (end 71.98 95.62) (width 0.5) (layer "B.Cu") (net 2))
 (segment (start 87.06 95.62) (end 79.05 95.62) (width 0.5) (layer "B.Cu") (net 2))
 (segment (start 91.39 64.407246) (end 91.39 49.88) (width 0.5) (layer "B.Cu") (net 2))
 (segment (start 89.303623 66.493623) (end 91.39 64.407246) (width 0.5) (layer "B.Cu") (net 2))
 (segment (start 89.303623 74.18) (end 89.303623 66.493623) (width 0.5) (layer "B.Cu") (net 2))
 (segment (start 79.05 84.433623) (end 89.303623 74.18) (width 0.5) (layer "B.Cu") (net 2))
 (segment (start 91.39 49.88) (end 87.13 45.62) (width 0.5) (layer "B.Cu") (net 2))
 (segment (start 79.05 95.62) (end 79.05 84.433623) (width 0.5) (layer "B.Cu") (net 2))
 (segment (start 87.13 45.62) (end 87.13 43.18) (width 0.5) (layer "B.Cu") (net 2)))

